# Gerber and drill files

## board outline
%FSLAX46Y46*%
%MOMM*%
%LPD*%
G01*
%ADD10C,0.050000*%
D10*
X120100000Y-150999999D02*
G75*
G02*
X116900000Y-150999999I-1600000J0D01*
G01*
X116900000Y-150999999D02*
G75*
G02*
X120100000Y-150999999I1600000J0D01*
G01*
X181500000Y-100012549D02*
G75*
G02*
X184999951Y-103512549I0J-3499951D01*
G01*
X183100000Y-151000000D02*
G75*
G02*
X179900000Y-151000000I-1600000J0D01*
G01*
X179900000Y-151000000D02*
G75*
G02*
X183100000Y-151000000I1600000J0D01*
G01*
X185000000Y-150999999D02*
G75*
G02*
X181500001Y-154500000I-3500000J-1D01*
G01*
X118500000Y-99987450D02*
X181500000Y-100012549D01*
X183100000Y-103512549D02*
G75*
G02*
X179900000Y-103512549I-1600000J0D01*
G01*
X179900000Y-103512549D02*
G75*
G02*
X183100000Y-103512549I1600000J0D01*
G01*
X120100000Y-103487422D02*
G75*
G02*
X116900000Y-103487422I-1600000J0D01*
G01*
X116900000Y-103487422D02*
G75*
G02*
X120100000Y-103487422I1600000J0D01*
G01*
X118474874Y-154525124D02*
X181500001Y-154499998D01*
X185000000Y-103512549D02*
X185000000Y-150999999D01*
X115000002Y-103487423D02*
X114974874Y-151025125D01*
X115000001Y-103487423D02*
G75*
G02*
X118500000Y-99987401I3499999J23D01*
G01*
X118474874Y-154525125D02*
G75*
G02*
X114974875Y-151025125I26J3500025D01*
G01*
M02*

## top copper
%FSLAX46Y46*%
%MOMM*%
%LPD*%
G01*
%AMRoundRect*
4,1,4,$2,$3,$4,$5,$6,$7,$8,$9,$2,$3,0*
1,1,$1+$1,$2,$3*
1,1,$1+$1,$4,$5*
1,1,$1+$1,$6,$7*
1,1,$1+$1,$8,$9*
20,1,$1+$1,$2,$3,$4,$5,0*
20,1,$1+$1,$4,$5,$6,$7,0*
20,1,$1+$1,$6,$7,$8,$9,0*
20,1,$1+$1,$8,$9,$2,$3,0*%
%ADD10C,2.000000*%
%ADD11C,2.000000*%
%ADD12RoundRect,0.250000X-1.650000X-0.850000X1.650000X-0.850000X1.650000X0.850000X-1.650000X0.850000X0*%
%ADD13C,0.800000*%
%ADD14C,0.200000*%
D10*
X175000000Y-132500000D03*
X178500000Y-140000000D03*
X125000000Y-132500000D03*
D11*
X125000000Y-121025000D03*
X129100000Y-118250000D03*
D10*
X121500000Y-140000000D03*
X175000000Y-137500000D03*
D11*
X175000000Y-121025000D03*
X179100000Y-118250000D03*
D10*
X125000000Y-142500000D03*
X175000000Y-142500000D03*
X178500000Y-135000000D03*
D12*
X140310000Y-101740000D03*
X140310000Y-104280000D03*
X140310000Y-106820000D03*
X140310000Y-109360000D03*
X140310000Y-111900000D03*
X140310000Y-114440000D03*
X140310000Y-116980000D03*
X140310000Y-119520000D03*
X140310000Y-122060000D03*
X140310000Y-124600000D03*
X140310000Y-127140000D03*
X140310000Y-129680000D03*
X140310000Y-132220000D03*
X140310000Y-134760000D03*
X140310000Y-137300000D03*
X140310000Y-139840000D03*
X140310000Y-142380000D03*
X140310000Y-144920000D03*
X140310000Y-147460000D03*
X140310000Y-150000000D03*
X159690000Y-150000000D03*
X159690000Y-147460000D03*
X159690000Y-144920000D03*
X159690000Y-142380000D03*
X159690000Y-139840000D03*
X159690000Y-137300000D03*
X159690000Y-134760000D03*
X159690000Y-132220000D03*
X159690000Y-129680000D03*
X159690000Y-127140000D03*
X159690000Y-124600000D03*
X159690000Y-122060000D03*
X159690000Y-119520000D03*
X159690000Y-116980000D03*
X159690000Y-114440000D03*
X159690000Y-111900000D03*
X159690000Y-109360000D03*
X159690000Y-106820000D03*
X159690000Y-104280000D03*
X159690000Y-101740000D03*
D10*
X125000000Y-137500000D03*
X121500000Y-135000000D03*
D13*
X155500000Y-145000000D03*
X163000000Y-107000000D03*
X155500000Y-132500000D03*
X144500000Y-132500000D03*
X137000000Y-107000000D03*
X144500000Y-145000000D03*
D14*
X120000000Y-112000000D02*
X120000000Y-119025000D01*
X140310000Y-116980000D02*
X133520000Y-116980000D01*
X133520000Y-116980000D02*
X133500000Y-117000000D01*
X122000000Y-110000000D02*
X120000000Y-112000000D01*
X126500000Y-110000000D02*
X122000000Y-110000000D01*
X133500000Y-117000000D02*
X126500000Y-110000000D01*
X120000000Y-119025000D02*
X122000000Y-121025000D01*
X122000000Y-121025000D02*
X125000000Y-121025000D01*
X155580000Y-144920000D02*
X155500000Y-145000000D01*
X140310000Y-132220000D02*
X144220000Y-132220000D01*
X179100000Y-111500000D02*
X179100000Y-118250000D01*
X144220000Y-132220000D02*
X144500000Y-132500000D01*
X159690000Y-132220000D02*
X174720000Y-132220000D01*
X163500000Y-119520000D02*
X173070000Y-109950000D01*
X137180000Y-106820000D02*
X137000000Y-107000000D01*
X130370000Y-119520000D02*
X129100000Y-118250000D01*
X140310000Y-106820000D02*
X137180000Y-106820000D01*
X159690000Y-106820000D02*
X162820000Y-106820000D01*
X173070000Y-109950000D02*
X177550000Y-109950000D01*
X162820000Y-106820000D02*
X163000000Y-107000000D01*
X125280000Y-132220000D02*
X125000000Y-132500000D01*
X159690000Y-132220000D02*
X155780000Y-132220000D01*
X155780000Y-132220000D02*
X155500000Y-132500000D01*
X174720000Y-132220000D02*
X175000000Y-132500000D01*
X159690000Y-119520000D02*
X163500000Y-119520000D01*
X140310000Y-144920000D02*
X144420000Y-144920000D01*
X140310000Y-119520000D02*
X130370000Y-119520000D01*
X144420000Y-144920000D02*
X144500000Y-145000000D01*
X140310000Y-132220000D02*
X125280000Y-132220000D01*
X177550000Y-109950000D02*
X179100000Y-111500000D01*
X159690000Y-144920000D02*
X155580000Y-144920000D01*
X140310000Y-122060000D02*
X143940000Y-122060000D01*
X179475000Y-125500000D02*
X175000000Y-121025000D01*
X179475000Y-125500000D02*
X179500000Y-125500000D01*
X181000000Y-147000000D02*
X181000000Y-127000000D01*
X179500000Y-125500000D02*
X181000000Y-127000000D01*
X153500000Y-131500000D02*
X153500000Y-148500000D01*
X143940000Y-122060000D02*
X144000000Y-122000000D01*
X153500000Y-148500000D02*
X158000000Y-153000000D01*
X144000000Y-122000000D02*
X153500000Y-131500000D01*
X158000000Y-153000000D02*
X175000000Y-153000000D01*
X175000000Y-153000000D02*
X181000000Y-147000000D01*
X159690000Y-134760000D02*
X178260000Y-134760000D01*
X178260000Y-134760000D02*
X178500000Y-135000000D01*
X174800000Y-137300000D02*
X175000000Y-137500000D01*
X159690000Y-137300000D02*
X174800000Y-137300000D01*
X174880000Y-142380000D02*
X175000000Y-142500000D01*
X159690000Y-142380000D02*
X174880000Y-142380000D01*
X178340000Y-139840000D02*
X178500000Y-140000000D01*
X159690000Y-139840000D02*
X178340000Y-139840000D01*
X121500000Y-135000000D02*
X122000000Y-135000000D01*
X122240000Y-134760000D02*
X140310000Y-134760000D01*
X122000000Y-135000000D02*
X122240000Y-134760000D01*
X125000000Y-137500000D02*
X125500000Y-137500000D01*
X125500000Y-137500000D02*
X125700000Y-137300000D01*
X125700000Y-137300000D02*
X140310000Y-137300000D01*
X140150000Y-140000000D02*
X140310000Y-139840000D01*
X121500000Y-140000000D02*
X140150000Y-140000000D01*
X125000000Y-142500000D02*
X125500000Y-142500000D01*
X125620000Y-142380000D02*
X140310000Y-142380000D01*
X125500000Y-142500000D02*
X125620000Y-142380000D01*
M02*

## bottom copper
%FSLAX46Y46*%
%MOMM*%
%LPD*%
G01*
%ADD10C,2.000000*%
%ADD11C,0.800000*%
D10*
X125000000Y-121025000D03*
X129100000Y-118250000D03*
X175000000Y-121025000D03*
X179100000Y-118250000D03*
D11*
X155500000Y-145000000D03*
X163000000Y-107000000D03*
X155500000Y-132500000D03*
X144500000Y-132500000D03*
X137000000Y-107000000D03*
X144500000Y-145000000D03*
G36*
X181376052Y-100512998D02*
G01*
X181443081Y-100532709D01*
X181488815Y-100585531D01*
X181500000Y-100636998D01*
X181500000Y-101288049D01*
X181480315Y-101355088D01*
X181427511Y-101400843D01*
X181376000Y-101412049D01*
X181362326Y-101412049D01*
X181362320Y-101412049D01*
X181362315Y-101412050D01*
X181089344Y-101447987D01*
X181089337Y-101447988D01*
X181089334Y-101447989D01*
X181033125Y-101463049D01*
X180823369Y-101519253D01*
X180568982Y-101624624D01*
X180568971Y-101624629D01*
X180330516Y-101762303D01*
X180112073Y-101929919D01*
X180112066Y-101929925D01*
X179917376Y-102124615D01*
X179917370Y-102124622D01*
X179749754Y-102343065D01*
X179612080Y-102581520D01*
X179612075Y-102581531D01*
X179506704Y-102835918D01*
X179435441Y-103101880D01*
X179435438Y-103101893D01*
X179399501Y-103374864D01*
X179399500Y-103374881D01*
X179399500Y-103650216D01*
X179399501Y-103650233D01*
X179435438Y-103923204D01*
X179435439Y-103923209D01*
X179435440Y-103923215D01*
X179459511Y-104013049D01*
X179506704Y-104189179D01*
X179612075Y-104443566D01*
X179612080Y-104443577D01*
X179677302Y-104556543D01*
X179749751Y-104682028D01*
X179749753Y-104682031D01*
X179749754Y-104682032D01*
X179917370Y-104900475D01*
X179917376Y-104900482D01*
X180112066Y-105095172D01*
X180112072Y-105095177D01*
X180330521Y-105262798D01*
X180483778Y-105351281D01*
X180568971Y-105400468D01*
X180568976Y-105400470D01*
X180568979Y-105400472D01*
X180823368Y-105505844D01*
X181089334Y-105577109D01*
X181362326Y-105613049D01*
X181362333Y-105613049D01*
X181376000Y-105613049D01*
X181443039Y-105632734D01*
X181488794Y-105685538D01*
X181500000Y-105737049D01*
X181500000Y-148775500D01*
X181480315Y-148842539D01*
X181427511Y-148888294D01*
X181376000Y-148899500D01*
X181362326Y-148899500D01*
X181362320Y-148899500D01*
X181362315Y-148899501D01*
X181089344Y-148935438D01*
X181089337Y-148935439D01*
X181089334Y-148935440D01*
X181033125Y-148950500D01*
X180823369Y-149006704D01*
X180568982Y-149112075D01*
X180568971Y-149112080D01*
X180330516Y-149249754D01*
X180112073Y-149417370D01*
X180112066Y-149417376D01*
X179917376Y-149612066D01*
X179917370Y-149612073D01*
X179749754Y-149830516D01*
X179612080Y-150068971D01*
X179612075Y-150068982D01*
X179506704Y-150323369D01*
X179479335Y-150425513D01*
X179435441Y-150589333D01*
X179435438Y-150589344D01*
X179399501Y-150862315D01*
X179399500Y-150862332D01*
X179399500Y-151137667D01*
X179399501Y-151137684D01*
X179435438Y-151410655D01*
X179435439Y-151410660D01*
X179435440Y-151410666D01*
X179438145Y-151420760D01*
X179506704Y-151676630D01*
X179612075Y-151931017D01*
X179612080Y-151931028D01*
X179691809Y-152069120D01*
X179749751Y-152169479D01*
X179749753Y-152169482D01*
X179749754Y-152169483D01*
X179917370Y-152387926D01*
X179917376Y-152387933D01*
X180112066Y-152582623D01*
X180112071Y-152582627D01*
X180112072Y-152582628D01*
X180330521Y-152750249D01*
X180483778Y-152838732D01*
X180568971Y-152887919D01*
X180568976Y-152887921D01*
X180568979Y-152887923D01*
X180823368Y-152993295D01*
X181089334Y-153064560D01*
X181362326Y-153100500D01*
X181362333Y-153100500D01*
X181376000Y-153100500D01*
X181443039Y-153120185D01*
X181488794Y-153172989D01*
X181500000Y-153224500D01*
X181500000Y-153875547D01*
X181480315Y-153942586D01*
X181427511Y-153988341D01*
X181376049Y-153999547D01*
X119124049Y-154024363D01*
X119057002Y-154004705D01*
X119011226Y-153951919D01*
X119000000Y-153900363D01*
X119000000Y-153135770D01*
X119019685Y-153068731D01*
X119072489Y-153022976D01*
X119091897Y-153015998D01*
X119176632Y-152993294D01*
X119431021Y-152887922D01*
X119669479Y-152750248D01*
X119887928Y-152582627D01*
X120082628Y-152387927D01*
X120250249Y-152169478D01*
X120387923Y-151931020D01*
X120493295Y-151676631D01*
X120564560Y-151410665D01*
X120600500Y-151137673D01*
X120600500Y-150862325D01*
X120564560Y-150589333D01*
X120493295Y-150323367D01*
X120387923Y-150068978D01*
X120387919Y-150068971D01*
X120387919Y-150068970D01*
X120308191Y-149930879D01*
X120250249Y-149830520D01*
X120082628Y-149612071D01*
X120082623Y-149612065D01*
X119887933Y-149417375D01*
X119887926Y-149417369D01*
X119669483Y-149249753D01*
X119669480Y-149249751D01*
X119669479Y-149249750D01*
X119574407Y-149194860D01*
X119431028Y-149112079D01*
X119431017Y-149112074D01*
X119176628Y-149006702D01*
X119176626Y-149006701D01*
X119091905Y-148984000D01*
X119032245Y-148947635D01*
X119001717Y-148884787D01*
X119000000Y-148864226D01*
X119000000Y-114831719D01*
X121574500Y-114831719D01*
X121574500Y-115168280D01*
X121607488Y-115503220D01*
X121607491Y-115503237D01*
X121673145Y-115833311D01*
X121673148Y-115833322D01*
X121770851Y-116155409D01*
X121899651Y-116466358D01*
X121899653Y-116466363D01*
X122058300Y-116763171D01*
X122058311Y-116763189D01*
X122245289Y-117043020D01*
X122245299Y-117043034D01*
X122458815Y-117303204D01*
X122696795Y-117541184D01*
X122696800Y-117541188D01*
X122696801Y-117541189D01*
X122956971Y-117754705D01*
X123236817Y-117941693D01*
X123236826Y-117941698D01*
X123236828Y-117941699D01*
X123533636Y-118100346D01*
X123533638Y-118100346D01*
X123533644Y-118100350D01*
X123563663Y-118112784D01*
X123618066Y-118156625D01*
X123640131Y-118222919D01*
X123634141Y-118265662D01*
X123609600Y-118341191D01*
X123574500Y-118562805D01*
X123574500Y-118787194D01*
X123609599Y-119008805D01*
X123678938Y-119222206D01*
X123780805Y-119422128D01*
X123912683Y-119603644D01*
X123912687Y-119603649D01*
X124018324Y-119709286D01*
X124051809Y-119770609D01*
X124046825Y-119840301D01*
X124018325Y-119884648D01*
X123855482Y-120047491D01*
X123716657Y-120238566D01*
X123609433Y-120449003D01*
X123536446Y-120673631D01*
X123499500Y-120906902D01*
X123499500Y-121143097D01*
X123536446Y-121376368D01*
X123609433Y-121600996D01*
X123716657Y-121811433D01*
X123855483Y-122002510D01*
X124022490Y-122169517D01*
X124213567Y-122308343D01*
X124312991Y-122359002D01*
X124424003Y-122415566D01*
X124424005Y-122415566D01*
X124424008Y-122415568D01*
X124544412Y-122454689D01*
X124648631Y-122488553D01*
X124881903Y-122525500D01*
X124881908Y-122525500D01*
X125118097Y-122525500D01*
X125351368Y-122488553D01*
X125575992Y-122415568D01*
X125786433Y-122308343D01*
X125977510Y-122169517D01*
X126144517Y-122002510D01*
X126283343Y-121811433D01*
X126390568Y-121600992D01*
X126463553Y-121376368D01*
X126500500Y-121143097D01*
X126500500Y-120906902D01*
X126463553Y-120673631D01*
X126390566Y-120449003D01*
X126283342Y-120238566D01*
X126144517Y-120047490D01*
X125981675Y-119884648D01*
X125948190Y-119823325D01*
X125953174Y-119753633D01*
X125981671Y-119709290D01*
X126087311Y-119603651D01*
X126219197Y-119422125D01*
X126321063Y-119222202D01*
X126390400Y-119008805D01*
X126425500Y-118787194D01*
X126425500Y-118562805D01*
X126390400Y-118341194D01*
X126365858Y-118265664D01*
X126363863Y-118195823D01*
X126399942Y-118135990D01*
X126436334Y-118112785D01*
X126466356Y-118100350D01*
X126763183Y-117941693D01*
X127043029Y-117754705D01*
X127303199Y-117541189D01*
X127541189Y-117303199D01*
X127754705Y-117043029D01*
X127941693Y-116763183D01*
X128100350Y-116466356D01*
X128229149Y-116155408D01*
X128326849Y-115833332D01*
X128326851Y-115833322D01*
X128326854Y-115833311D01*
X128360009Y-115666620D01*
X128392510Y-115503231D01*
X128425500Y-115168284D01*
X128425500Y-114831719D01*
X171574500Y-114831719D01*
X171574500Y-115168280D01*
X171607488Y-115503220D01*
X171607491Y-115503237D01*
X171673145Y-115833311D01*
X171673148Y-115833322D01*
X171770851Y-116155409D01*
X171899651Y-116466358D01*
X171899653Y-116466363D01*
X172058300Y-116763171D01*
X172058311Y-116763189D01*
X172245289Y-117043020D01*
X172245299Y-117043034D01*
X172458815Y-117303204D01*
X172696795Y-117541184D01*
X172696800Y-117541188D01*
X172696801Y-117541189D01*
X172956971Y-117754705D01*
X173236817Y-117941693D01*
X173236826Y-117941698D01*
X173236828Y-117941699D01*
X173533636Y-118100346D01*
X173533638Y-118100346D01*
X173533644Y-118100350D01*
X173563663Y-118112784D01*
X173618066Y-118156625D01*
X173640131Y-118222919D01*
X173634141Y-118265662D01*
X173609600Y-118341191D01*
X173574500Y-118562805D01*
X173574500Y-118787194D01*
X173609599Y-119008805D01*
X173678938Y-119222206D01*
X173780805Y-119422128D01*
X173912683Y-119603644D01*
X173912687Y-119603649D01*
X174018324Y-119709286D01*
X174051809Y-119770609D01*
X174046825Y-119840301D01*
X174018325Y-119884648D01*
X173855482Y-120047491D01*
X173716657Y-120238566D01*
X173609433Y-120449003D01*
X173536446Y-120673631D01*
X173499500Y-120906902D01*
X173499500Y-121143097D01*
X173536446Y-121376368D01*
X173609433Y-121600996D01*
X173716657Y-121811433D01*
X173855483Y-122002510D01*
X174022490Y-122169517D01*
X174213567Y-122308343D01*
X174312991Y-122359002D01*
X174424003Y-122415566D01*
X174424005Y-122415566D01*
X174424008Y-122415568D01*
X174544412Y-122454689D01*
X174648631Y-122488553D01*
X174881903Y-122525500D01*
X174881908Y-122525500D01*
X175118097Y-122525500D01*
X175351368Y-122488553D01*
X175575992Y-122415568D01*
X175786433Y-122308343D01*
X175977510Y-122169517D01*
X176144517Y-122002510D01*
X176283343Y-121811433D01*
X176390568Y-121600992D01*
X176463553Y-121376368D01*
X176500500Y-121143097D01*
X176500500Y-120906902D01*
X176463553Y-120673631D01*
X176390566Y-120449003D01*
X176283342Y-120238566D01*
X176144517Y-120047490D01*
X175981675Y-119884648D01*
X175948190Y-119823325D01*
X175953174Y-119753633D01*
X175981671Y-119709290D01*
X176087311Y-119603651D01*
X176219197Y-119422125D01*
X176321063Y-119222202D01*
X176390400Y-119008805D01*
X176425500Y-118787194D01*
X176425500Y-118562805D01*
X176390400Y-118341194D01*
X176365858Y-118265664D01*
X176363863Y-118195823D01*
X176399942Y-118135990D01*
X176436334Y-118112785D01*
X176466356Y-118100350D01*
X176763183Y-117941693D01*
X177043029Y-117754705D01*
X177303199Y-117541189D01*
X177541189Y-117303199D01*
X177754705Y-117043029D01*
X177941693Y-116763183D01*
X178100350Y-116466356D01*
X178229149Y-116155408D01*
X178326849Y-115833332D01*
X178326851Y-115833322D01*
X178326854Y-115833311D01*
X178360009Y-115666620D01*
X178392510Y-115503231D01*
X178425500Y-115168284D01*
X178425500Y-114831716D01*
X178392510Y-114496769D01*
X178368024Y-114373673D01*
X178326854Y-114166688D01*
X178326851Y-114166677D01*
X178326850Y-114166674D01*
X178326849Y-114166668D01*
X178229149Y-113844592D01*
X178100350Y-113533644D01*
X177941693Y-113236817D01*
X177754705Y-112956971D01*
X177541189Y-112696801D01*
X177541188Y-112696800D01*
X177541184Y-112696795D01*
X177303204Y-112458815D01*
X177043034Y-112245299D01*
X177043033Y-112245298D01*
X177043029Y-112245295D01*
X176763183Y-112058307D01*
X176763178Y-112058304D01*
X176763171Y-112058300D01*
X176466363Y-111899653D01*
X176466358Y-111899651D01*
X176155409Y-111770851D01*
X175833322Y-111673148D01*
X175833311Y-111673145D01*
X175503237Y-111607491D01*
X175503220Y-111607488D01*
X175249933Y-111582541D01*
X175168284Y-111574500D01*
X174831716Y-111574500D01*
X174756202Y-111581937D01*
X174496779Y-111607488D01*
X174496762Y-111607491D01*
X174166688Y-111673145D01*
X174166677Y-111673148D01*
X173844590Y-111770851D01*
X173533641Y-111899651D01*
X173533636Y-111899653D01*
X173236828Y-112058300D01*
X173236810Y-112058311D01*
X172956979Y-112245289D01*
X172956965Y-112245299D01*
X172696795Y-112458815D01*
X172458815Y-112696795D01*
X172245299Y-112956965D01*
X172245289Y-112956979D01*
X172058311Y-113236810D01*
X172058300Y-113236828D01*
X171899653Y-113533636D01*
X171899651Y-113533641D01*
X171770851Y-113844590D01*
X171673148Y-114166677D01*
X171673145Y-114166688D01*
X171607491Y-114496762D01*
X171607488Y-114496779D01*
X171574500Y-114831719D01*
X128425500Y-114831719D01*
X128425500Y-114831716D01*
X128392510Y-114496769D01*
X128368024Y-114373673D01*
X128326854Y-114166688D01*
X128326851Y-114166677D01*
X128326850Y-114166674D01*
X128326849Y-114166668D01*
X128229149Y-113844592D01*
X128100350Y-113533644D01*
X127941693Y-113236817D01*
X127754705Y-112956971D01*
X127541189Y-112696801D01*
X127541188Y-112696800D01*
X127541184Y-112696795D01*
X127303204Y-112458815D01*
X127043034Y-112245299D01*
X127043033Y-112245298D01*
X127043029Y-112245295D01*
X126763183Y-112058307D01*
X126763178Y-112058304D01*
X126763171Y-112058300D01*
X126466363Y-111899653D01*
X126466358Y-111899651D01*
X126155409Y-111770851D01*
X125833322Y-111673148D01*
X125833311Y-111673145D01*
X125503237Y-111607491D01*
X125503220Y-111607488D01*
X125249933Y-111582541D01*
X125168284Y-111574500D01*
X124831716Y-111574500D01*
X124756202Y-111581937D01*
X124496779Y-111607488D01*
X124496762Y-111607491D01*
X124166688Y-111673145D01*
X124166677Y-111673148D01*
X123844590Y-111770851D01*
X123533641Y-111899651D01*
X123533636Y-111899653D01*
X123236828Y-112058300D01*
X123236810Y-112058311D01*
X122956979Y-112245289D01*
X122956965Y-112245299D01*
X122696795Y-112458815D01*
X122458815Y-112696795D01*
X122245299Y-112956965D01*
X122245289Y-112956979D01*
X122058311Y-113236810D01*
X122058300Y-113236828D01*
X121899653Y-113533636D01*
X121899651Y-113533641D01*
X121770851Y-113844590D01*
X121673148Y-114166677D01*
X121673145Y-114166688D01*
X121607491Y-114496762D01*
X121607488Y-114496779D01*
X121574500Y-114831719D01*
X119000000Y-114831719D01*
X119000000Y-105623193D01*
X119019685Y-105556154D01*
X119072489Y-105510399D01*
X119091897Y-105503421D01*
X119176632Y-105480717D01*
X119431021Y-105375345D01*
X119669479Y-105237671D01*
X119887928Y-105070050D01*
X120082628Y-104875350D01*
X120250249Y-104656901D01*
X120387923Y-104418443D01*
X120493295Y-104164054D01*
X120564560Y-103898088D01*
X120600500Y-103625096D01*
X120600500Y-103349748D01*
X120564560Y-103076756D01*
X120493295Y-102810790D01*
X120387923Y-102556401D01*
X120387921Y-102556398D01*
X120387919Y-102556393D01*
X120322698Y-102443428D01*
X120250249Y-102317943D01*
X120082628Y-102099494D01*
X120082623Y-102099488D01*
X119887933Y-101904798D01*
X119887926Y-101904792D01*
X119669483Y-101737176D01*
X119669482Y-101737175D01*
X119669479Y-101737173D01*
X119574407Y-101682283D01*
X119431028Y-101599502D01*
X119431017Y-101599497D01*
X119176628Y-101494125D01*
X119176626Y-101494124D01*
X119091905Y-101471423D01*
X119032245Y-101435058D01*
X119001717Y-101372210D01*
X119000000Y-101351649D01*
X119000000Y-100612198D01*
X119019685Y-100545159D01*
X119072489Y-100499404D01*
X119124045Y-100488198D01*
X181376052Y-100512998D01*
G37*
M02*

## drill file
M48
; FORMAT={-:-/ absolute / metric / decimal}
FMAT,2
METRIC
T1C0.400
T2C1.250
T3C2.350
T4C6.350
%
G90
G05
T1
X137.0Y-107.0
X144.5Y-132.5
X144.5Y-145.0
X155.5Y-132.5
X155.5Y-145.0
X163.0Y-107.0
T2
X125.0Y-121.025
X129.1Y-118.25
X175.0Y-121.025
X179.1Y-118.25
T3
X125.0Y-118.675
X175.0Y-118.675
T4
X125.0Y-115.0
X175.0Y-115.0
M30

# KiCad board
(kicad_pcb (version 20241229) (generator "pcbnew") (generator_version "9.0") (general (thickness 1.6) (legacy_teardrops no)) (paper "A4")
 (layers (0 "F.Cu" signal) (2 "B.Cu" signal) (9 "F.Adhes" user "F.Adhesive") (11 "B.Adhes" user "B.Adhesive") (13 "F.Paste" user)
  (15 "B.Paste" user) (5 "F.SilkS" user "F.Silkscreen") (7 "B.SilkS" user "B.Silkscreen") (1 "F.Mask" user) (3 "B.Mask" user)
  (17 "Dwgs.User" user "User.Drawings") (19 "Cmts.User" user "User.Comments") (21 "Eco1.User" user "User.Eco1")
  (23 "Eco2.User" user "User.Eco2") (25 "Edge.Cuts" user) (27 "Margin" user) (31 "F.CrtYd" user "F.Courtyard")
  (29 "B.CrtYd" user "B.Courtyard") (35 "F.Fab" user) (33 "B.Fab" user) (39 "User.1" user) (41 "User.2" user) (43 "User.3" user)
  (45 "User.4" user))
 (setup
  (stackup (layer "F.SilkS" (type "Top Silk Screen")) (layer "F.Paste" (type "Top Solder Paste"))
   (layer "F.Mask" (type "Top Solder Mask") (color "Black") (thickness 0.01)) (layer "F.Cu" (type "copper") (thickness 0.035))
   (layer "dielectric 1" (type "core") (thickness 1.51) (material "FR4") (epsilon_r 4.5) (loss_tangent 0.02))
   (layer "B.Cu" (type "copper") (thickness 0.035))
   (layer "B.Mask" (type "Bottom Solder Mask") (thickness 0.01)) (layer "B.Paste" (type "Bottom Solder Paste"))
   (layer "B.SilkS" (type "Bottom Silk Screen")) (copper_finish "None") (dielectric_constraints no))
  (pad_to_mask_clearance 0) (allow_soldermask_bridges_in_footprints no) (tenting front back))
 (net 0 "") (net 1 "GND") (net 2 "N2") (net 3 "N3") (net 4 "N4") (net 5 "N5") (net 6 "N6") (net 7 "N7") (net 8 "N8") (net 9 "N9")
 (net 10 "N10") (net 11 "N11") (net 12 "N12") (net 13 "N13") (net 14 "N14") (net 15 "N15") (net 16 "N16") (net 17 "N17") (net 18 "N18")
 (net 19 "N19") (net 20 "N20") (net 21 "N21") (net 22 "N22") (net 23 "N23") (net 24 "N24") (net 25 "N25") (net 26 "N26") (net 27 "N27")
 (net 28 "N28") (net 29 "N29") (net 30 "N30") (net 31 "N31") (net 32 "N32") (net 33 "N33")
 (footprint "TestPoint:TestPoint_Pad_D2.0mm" (layer "F.Cu") (at 175 132.5)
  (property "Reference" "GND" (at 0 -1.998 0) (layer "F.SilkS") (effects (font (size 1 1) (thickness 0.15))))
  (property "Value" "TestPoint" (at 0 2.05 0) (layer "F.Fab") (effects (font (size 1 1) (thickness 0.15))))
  (pad "1" smd circle (at 0 0) (size 2 2) (layers "F.Cu" "F.Mask") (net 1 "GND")))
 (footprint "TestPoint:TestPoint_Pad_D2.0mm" (layer "F.Cu") (at 178.5 140)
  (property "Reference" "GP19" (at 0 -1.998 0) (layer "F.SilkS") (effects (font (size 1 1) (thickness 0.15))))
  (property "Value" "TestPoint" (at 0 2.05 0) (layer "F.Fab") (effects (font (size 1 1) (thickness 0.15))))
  (pad "1" smd circle (at 0 0) (size 2 2) (layers "F.Cu" "F.Mask") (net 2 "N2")))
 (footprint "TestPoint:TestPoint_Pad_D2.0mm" (layer "F.Cu") (at 125 132.5)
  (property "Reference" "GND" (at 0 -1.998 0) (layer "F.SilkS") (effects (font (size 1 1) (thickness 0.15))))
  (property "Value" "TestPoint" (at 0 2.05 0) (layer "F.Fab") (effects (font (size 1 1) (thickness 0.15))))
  (pad "1" smd circle (at 0 0) (size 2 2) (layers "F.Cu" "F.Mask") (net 1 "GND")))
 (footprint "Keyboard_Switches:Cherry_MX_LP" (layer "F.Cu") (at 125 115)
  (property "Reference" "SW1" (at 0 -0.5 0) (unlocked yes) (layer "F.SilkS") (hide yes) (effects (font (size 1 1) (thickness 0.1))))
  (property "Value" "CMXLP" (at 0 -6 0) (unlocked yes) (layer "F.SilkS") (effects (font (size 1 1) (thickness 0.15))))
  (pad "" np_thru_hole circle (at 0 0) (size 6.35 6.35) (drill 6.35) (layers "*.Cu" "*.Mask"))
  (pad "" np_thru_hole circle (at 0 3.675) (size 2.35 2.35) (drill 2.35) (layers "*.Cu" "*.Mask"))
  (pad "1" thru_hole circle (at 0 6.025) (size 2 2) (drill 1.25) (layers "*.Cu" "*.Mask") (remove_unused_layers no) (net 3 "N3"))
  (pad "2" thru_hole circle (at 4.1 3.25) (size 2 2) (drill 1.25) (layers "*.Cu" "*.Mask") (remove_unused_layers no) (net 1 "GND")))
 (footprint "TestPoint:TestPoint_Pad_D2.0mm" (layer "F.Cu") (at 121.5 140)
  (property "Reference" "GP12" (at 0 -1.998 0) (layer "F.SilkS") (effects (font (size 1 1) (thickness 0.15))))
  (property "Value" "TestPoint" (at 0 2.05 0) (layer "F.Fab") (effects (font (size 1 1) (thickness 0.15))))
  (pad "1" smd circle (at 0 0) (size 2 2) (layers "F.Cu" "F.Mask") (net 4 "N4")))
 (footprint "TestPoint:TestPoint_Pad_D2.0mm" (layer "F.Cu") (at 175 137.5)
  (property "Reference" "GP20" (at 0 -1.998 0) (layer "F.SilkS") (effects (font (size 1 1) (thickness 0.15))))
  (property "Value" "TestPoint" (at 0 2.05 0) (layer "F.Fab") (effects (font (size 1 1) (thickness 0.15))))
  (pad "1" smd circle (at 0 0) (size 2 2) (layers "F.Cu" "F.Mask") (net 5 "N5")))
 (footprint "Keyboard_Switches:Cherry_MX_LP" (layer "F.Cu") (at 175 115)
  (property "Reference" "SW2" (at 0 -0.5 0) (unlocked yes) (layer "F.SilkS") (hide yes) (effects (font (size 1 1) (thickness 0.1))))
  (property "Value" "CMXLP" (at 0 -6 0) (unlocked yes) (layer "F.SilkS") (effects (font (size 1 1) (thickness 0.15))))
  (pad "" np_thru_hole circle (at 0 0) (size 6.35 6.35) (drill 6.35) (layers "*.Cu" "*.Mask"))
  (pad "" np_thru_hole circle (at 0 3.675) (size 2.35 2.35) (drill 2.35) (layers "*.Cu" "*.Mask"))
  (pad "1" thru_hole circle (at 0 6.025) (size 2 2) (drill 1.25) (layers "*.Cu" "*.Mask") (remove_unused_layers no) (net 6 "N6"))
  (pad "2" thru_hole circle (at 4.1 3.25) (size 2 2) (drill 1.25) (layers "*.Cu" "*.Mask") (remove_unused_layers no) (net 1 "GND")))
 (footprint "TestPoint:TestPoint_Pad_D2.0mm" (layer "F.Cu") (at 125 142.5)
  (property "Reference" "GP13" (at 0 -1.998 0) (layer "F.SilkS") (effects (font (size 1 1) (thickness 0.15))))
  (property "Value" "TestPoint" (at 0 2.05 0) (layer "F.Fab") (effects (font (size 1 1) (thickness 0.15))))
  (pad "1" smd circle (at 0 0) (size 2 2) (layers "F.Cu" "F.Mask") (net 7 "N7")))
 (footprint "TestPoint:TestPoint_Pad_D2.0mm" (layer "F.Cu") (at 175 142.5)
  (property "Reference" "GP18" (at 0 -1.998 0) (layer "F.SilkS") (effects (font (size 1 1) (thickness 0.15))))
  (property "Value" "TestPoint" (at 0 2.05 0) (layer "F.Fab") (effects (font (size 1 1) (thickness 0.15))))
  (pad "1" smd circle (at 0 0) (size 2 2) (layers "F.Cu" "F.Mask") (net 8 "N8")))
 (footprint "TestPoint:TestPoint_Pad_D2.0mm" (layer "F.Cu") (at 178.5 135)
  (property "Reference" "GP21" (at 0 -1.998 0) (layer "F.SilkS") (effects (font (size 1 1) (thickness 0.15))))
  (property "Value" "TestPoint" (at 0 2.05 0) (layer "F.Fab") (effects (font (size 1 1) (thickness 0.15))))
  (pad "1" smd circle (at 0 0) (size 2 2) (layers "F.Cu" "F.Mask") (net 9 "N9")))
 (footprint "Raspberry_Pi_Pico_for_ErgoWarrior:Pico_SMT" (layer "F.Cu") (at 150 150)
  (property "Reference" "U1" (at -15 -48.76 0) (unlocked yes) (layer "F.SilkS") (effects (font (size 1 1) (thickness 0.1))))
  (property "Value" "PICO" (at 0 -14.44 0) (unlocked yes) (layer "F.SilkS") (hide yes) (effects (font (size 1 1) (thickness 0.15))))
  (pad "1" smd roundrect (at -9.69 -48.26) (size 3.8 2.2) (layers "F.Cu" "F.Mask" "F.Paste") (roundrect_rratio 0.1136363636) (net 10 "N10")
   (thermal_bridge_angle 45))
  (pad "2" smd roundrect (at -9.69 -45.72) (size 3.8 2.2) (layers "F.Cu" "F.Mask" "F.Paste") (roundrect_rratio 0.1136363636) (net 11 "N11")
   (thermal_bridge_angle 45))
  (pad "3" smd roundrect (at -9.69 -43.18) (size 3.8 2.2) (layers "F.Cu" "F.Mask" "F.Paste") (roundrect_rratio 0.1136363636) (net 1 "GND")
   (thermal_bridge_angle 45))
  (pad "4" smd roundrect (at -9.69 -40.64) (size 3.8 2.2) (layers "F.Cu" "F.Mask" "F.Paste") (roundrect_rratio 0.1136363636) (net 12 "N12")
   (thermal_bridge_angle 45))
  (pad "5" smd roundrect (at -9.69 -38.1) (size 3.8 2.2) (layers "F.Cu" "F.Mask" "F.Paste") (roundrect_rratio 0.1136363636) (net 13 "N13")
   (thermal_bridge_angle 45))
  (pad "6" smd roundrect (at -9.69 -35.56) (size 3.8 2.2) (layers "F.Cu" "F.Mask" "F.Paste") (roundrect_rratio 0.1136363636) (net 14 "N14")
   (thermal_bridge_angle 45))
  (pad "7" smd roundrect (at -9.69 -33.02) (size 3.8 2.2) (layers "F.Cu" "F.Mask" "F.Paste") (roundrect_rratio 0.1136363636) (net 3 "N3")
   (thermal_bridge_angle 45))
  (pad "8" smd roundrect (at -9.69 -30.48) (size 3.8 2.2) (layers "F.Cu" "F.Mask" "F.Paste") (roundrect_rratio 0.1136363636) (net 1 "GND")
   (thermal_bridge_angle 45))
  (pad "9" smd roundrect (at -9.69 -27.94) (size 3.8 2.2) (layers "F.Cu" "F.Mask" "F.Paste") (roundrect_rratio 0.1136363636) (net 6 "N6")
   (thermal_bridge_angle 45))
  (pad "10" smd roundrect (at -9.69 -25.4) (size 3.8 2.2) (layers "F.Cu" "F.Mask" "F.Paste") (roundrect_rratio 0.1136363636) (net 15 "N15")
   (thermal_bridge_angle 45))
  (pad "11" smd roundrect (at -9.69 -22.86) (size 3.8 2.2) (layers "F.Cu" "F.Mask" "F.Paste") (roundrect_rratio 0.1136363636) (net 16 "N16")
   (thermal_bridge_angle 45))
  (pad "12" smd roundrect (at -9.69 -20.32) (size 3.8 2.2) (layers "F.Cu" "F.Mask" "F.Paste") (roundrect_rratio 0.1136363636) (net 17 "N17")
   (thermal_bridge_angle 45))
  (pad "13" smd roundrect (at -9.69 -17.78) (size 3.8 2.2) (layers "F.Cu" "F.Mask" "F.Paste") (roundrect_rratio 0.1136363636) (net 1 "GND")
   (thermal_bridge_angle 45))
  (pad "14" smd roundrect (at -9.69 -15.24) (size 3.8 2.2) (layers "F.Cu" "F.Mask" "F.Paste") (roundrect_rratio 0.1136363636) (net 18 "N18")
   (thermal_bridge_angle 45))
  (pad "15" smd roundrect (at -9.69 -12.7) (size 3.8 2.2) (layers "F.Cu" "F.Mask" "F.Paste") (roundrect_rratio 0.1136363636) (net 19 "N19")
   (thermal_bridge_angle 45))
  (pad "16" smd roundrect (at -9.69 -10.16) (size 3.8 2.2) (layers "F.Cu" "F.Mask" "F.Paste") (roundrect_rratio 0.1136363636) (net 4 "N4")
   (thermal_bridge_angle 45))
  (pad "17" smd roundrect (at -9.69 -7.62) (size 3.8 2.2) (layers "F.Cu" "F.Mask" "F.Paste") (roundrect_rratio 0.1136363636) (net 7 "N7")
   (thermal_bridge_angle 45))
  (pad "18" smd roundrect (at -9.69 -5.08) (size 3.8 2.2) (layers "F.Cu" "F.Mask" "F.Paste") (roundrect_rratio 0.1136363636) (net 1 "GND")
   (thermal_bridge_angle 45))
  (pad "19" smd roundrect (at -9.69 -2.54) (size 3.8 2.2) (layers "F.Cu" "F.Mask" "F.Paste") (roundrect_rratio 0.1136363636) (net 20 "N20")
   (thermal_bridge_angle 45))
  (pad "20" smd roundrect (at -9.69 0) (size 3.8 2.2) (layers "F.Cu" "F.Mask" "F.Paste") (roundrect_rratio 0.1136363636) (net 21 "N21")
   (thermal_bridge_angle 45))
  (pad "21" smd roundrect (at 9.69 0) (size 3.8 2.2) (layers "F.Cu" "F.Mask" "F.Paste") (roundrect_rratio 0.1136363636) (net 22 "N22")
   (thermal_bridge_angle 45))
  (pad "22" smd roundrect (at 9.69 -2.54) (size 3.8 2.2) (layers "F.Cu" "F.Mask" "F.Paste") (roundrect_rratio 0.1136363636) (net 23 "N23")
   (thermal_bridge_angle 45))
  (pad "23" smd roundrect (at 9.69 -5.08) (size 3.8 2.2) (layers "F.Cu" "F.Mask" "F.Paste") (roundrect_rratio 0.1136363636) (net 1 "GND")
   (thermal_bridge_angle 45))
  (pad "24" smd roundrect (at 9.69 -7.62) (size 3.8 2.2) (layers "F.Cu" "F.Mask" "F.Paste") (roundrect_rratio 0.1136363636) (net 8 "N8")
   (thermal_bridge_angle 45))
  (pad "25" smd roundrect (at 9.69 -10.16) (size 3.8 2.2) (layers "F.Cu" "F.Mask" "F.Paste") (roundrect_rratio 0.1136363636) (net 2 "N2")
   (thermal_bridge_angle 45))
  (pad "26" smd roundrect (at 9.69 -12.7) (size 3.8 2.2) (layers "F.Cu" "F.Mask" "F.Paste") (roundrect_rratio 0.1136363636) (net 5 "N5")
   (thermal_bridge_angle 45))
  (pad "27" smd roundrect (at 9.69 -15.24) (size 3.8 2.2) (layers "F.Cu" "F.Mask" "F.Paste") (roundrect_rratio 0.1136363636) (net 9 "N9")
   (thermal_bridge_angle 45))
  (pad "28" smd roundrect (at 9.69 -17.78) (size 3.8 2.2) (layers "F.Cu" "F.Mask" "F.Paste") (roundrect_rratio 0.1136363636) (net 1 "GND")
   (thermal_bridge_angle 45))
  (pad "29" smd roundrect (at 9.69 -20.32) (size 3.8 2.2) (layers "F.Cu" "F.Mask" "F.Paste") (roundrect_rratio 0.1136363636) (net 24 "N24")
   (thermal_bridge_angle 45))
  (pad "30" smd roundrect (at 9.69 -22.86) (size 3.8 2.2) (layers "F.Cu" "F.Mask" "F.Paste") (roundrect_rratio 0.1136363636) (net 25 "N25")
   (thermal_bridge_angle 45))
  (pad "31" smd roundrect (at 9.69 -25.4) (size 3.8 2.2) (layers "F.Cu" "F.Mask" "F.Paste") (roundrect_rratio 0.1136363636) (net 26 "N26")
   (thermal_bridge_angle 45))
  (pad "32" smd roundrect (at 9.69 -27.94) (size 3.8 2.2) (layers "F.Cu" "F.Mask" "F.Paste") (roundrect_rratio 0.1136363636) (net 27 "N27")
   (thermal_bridge_angle 45))
  (pad "33" smd roundrect (at 9.69 -30.48) (size 3.8 2.2) (layers "F.Cu" "F.Mask" "F.Paste") (roundrect_rratio 0.1136363636) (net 1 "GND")
   (thermal_bridge_angle 45))
  (pad "34" smd roundrect (at 9.69 -33.02) (size 3.8 2.2) (layers "F.Cu" "F.Mask" "F.Paste") (roundrect_rratio 0.1136363636) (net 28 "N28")
   (thermal_bridge_angle 45))
  (pad "35" smd roundrect (at 9.69 -35.56) (size 3.8 2.2) (layers "F.Cu" "F.Mask" "F.Paste") (roundrect_rratio 0.1136363636) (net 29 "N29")
   (thermal_bridge_angle 45))
  (pad "36" smd roundrect (at 9.69 -38.1) (size 3.8 2.2) (layers "F.Cu" "F.Mask" "F.Paste") (roundrect_rratio 0.1136363636) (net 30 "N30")
   (thermal_bridge_angle 45))
  (pad "37" smd roundrect (at 9.69 -40.64) (size 3.8 2.2) (layers "F.Cu" "F.Mask" "F.Paste") (roundrect_rratio 0.1136363636) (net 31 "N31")
   (thermal_bridge_angle 45))
  (pad "38" smd roundrect (at 9.69 -43.18) (size 3.8 2.2) (layers "F.Cu" "F.Mask" "F.Paste") (roundrect_rratio 0.1136363636) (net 1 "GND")
   (thermal_bridge_angle 45))
  (pad "39" smd roundrect (at 9.69 -45.72) (size 3.8 2.2) (layers "F.Cu" "F.Mask" "F.Paste") (roundrect_rratio 0.1136363636) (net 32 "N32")
   (thermal_bridge_angle 45))
  (pad "40" smd roundrect (at 9.69 -48.26) (size 3.8 2.2) (layers "F.Cu" "F.Mask" "F.Paste") (roundrect_rratio 0.1136363636) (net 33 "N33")
   (thermal_bridge_angle 45)))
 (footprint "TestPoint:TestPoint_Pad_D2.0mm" (layer "F.Cu") (at 125 137.5)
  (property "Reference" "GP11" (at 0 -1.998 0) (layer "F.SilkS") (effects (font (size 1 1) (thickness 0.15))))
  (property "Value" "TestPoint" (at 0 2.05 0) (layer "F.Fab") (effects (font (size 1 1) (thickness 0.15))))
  (pad "1" smd circle (at 0 0) (size 2 2) (layers "F.Cu" "F.Mask") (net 19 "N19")))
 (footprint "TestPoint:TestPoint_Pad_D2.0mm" (layer "F.Cu") (at 121.5 135)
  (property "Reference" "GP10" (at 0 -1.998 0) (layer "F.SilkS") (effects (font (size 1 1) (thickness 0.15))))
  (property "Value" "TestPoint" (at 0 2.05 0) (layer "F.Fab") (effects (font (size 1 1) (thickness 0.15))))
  (pad "1" smd circle (at 0 0) (size 2 2) (layers "F.Cu" "F.Mask") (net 18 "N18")))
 (gr_circle (center 118.5 150.999999) (end 120.1 150.999999) (stroke (width 0.05) (type solid)) (fill no) (layer "Edge.Cuts"))
 (gr_arc (start 181.5 100.012549) (mid 183.974874 101.037675) (end 185 103.512549) (stroke (width 0.05) (type default)) (layer "Edge.Cuts"))
 (gr_circle (center 181.5 151) (end 183.1 151) (stroke (width 0.05) (type solid)) (fill no) (layer "Edge.Cuts"))
 (gr_arc (start 185 150.999999) (mid 183.974874 153.474872) (end 181.500001 154.499998) (stroke (width 0.05) (type default))
  (layer "Edge.Cuts"))
 (gr_line (start 118.5 99.98745) (end 181.5 100.012549) (stroke (width 0.05) (type default)) (layer "Edge.Cuts"))
 (gr_circle (center 181.5 103.512549) (end 183.1 103.512549) (stroke (width 0.05) (type solid)) (fill no) (layer "Edge.Cuts"))
 (gr_circle (center 118.5 103.487422) (end 120.1 103.487422) (stroke (width 0.05) (type solid)) (fill no) (layer "Edge.Cuts"))
 (gr_line (start 118.474874 154.525124) (end 181.500001 154.499998) (stroke (width 0.05) (type default)) (layer "Edge.Cuts"))
 (gr_line (start 185 103.512549) (end 185 150.999999) (stroke (width 0.05) (type default)) (layer "Edge.Cuts"))
 (gr_line (start 115.000002 103.487423) (end 114.974874 151.025125) (stroke (width 0.05) (type default)) (layer "Edge.Cuts"))
 (gr_arc (start 115.000001 103.487423) (mid 116.025127 101.01255) (end 118.5 99.987424) (stroke (width 0.05) (type default))
  (layer "Edge.Cuts"))
 (gr_arc (start 118.474874 154.525125) (mid 116 153.499999) (end 114.974874 151.025125) (stroke (width 0.05) (type solid))
  (layer "Edge.Cuts"))
 (segment (start 120 112) (end 120 119.025) (width 0.2) (layer "F.Cu") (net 3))
 (segment (start 140.31 116.98) (end 133.52 116.98) (width 0.2) (layer "F.Cu") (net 3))
 (segment (start 133.52 116.98) (end 133.5 117) (width 0.2) (layer "F.Cu") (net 3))
 (segment (start 122 110) (end 120 112) (width 0.2) (layer "F.Cu") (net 3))
 (segment (start 126.5 110) (end 122 110) (width 0.2) (layer "F.Cu") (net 3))
 (segment (start 133.5 117) (end 126.5 110) (width 0.2) (layer "F.Cu") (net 3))
 (segment (start 120 119.025) (end 122 121.025) (width 0.2) (layer "F.Cu") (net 3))
 (segment (start 122 121.025) (end 125 121.025) (width 0.2) (layer "F.Cu") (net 3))
 (segment (start 155.58 144.92) (end 155.5 145) (width 0.2) (layer "F.Cu") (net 1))
 (segment (start 140.31 132.22) (end 144.22 132.22) (width 0.2) (layer "F.Cu") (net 1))
 (segment (start 179.1 111.5) (end 179.1 118.25) (width 0.2) (layer "F.Cu") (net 1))
 (segment (start 144.22 132.22) (end 144.5 132.5) (width 0.2) (layer "F.Cu") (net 1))
 (segment (start 159.69 132.22) (end 174.72 132.22) (width 0.2) (layer "F.Cu") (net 1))
 (segment (start 163.5 119.52) (end 173.07 109.95) (width 0.2) (layer "F.Cu") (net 1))
 (segment (start 137.18 106.82) (end 137 107) (width 0.2) (layer "F.Cu") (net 1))
 (segment (start 130.37 119.52) (end 129.1 118.25) (width 0.2) (layer "F.Cu") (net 1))
 (segment (start 140.31 106.82) (end 137.18 106.82) (width 0.2) (layer "F.Cu") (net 1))
 (segment (start 159.69 106.82) (end 162.82 106.82) (width 0.2) (layer "F.Cu") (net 1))
 (segment (start 173.07 109.95) (end 177.55 109.95) (width 0.2) (layer "F.Cu") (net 1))
 (segment (start 162.82 106.82) (end 163 107) (width 0.2) (layer "F.Cu") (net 1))
 (segment (start 125.28 132.22) (end 125 132.5) (width 0.2) (layer "F.Cu") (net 1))
 (segment (start 159.69 132.22) (end 155.78 132.22) (width 0.2) (layer "F.Cu") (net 1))
 (segment (start 155.78 132.22) (end 155.5 132.5) (width 0.2) (layer "F.Cu") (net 1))
 (segment (start 174.72 132.22) (end 175 132.5) (width 0.2) (layer "F.Cu") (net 1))
 (segment (start 159.69 119.52) (end 163.5 119.52) (width 0.2) (layer "F.Cu") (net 1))
 (segment (start 140.31 144.92) (end 144.42 144.92) (width 0.2) (layer "F.Cu") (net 1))
 (segment (start 140.31 119.52) (end 130.37 119.52) (width 0.2) (layer "F.Cu") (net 1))
 (segment (start 144.42 144.92) (end 144.5 145) (width 0.2) (layer "F.Cu") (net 1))
 (segment (start 140.31 132.22) (end 125.28 132.22) (width 0.2) (layer "F.Cu") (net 1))
 (segment (start 177.55 109.95) (end 179.1 111.5) (width 0.2) (layer "F.Cu") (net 1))
 (segment (start 159.69 144.92) (end 155.58 144.92) (width 0.2) (layer "F.Cu") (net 1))
 (via (at 155.5 145) (size 0.8) (drill 0.4) (layers "F.Cu" "B.Cu") (free yes) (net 1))
 (via (at 163 107) (size 0.8) (drill 0.4) (layers "F.Cu" "B.Cu") (free yes) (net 1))
 (via (at 155.5 132.5) (size 0.8) (drill 0.4) (layers "F.Cu" "B.Cu") (free yes) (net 1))
 (via (at 144.5 132.5) (size 0.8) (drill 0.4) (layers "F.Cu" "B.Cu") (free yes) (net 1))
 (via (at 137 107) (size 0.8) (drill 0.4) (layers "F.Cu" "B.Cu") (free yes) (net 1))
 (via (at 144.5 145) (size 0.8) (drill 0.4) (layers "F.Cu" "B.Cu") (free yes) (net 1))
 (segment (start 140.31 122.06) (end 143.94 122.06) (width 0.2) (layer "F.Cu") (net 6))
 (segment (start 179.475 125.5) (end 175 121.025) (width 0.2) (layer "F.Cu") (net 6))
 (segment (start 179.475 125.5) (end 179.5 125.5) (width 0.2) (layer "F.Cu") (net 6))
 (segment (start 181 147) (end 181 127) (width 0.2) (layer "F.Cu") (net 6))
 (segment (start 179.5 125.5) (end 181 127) (width 0.2) (layer "F.Cu") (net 6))
 (segment (start 153.5 131.5) (end 153.5 148.5) (width 0.2) (layer "F.Cu") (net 6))
 (segment (start 143.94 122.06) (end 144 122) (width 0.2) (layer "F.Cu") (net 6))
 (segment (start 153.5 148.5) (end 158 153) (width 0.2) (layer "F.Cu") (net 6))
 (segment (start 144 122) (end 153.5 131.5) (width 0.2) (layer "F.Cu") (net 6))
 (segment (start 158 153) (end 175 153) (width 0.2) (layer "F.Cu") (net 6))
 (segment (start 175 153) (end 181 147) (width 0.2) (layer "F.Cu") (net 6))
 (segment (start 159.69 134.76) (end 178.26 134.76) (width 0.2) (layer "F.Cu") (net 9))
 (segment (start 178.26 134.76) (end 178.5 135) (width 0.2) (layer "F.Cu") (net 9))
 (segment (start 174.8 137.3) (end 175 137.5) (width 0.2) (layer "F.Cu") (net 5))
 (segment (start 159.69 137.3) (end 174.8 137.3) (width 0.2) (layer "F.Cu") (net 5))
 (segment (start 174.88 142.38) (end 175 142.5) (width 0.2) (layer "F.Cu") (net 8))
 (segment (start 159.69 142.38) (end 174.88 142.38) (width 0.2) (layer "F.Cu") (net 8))
 (segment (start 178.34 139.84) (end 178.5 140) (width 0.2) (layer "F.Cu") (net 2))
 (segment (start 159.69 139.84) (end 178.34 139.84) (width 0.2) (layer "F.Cu") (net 2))
 (segment (start 121.5 135) (end 122 135) (width 0.2) (layer "F.Cu") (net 18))
 (segment (start 122.24 134.76) (end 140.31 134.76) (width 0.2) (layer "F.Cu") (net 18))
 (segment (start 122 135) (end 122.24 134.76) (width 0.2) (layer "F.Cu") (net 18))
 (segment (start 125 137.5) (end 125.5 137.5) (width 0.2) (layer "F.Cu") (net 19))
 (segment (start 125.5 137.5) (end 125.7 137.3) (width 0.2) (layer "F.Cu") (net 19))
 (segment (start 125.7 137.3) (end 140.31 137.3) (width 0.2) (layer "F.Cu") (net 19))
 (segment (start 140.15 140) (end 140.31 139.84) (width 0.2) (layer "F.Cu") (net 4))
 (segment (start 121.5 140) (end 140.15 140) (width 0.2) (layer "F.Cu") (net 4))
 (segment (start 125 142.5) (end 125.5 142.5) (width 0.2) (layer "F.Cu") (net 7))
 (segment (start 125.62 142.38) (end 140.31 142.38) (width 0.2) (layer "F.Cu") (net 7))
 (segment (start 125.5 142.5) (end 125.62 142.38) (width 0.2) (layer "F.Cu") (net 7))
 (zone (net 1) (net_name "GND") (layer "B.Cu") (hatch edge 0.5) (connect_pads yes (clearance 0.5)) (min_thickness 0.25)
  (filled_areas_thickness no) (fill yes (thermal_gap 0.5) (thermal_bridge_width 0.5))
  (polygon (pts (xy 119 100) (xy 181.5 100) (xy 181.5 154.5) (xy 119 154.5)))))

